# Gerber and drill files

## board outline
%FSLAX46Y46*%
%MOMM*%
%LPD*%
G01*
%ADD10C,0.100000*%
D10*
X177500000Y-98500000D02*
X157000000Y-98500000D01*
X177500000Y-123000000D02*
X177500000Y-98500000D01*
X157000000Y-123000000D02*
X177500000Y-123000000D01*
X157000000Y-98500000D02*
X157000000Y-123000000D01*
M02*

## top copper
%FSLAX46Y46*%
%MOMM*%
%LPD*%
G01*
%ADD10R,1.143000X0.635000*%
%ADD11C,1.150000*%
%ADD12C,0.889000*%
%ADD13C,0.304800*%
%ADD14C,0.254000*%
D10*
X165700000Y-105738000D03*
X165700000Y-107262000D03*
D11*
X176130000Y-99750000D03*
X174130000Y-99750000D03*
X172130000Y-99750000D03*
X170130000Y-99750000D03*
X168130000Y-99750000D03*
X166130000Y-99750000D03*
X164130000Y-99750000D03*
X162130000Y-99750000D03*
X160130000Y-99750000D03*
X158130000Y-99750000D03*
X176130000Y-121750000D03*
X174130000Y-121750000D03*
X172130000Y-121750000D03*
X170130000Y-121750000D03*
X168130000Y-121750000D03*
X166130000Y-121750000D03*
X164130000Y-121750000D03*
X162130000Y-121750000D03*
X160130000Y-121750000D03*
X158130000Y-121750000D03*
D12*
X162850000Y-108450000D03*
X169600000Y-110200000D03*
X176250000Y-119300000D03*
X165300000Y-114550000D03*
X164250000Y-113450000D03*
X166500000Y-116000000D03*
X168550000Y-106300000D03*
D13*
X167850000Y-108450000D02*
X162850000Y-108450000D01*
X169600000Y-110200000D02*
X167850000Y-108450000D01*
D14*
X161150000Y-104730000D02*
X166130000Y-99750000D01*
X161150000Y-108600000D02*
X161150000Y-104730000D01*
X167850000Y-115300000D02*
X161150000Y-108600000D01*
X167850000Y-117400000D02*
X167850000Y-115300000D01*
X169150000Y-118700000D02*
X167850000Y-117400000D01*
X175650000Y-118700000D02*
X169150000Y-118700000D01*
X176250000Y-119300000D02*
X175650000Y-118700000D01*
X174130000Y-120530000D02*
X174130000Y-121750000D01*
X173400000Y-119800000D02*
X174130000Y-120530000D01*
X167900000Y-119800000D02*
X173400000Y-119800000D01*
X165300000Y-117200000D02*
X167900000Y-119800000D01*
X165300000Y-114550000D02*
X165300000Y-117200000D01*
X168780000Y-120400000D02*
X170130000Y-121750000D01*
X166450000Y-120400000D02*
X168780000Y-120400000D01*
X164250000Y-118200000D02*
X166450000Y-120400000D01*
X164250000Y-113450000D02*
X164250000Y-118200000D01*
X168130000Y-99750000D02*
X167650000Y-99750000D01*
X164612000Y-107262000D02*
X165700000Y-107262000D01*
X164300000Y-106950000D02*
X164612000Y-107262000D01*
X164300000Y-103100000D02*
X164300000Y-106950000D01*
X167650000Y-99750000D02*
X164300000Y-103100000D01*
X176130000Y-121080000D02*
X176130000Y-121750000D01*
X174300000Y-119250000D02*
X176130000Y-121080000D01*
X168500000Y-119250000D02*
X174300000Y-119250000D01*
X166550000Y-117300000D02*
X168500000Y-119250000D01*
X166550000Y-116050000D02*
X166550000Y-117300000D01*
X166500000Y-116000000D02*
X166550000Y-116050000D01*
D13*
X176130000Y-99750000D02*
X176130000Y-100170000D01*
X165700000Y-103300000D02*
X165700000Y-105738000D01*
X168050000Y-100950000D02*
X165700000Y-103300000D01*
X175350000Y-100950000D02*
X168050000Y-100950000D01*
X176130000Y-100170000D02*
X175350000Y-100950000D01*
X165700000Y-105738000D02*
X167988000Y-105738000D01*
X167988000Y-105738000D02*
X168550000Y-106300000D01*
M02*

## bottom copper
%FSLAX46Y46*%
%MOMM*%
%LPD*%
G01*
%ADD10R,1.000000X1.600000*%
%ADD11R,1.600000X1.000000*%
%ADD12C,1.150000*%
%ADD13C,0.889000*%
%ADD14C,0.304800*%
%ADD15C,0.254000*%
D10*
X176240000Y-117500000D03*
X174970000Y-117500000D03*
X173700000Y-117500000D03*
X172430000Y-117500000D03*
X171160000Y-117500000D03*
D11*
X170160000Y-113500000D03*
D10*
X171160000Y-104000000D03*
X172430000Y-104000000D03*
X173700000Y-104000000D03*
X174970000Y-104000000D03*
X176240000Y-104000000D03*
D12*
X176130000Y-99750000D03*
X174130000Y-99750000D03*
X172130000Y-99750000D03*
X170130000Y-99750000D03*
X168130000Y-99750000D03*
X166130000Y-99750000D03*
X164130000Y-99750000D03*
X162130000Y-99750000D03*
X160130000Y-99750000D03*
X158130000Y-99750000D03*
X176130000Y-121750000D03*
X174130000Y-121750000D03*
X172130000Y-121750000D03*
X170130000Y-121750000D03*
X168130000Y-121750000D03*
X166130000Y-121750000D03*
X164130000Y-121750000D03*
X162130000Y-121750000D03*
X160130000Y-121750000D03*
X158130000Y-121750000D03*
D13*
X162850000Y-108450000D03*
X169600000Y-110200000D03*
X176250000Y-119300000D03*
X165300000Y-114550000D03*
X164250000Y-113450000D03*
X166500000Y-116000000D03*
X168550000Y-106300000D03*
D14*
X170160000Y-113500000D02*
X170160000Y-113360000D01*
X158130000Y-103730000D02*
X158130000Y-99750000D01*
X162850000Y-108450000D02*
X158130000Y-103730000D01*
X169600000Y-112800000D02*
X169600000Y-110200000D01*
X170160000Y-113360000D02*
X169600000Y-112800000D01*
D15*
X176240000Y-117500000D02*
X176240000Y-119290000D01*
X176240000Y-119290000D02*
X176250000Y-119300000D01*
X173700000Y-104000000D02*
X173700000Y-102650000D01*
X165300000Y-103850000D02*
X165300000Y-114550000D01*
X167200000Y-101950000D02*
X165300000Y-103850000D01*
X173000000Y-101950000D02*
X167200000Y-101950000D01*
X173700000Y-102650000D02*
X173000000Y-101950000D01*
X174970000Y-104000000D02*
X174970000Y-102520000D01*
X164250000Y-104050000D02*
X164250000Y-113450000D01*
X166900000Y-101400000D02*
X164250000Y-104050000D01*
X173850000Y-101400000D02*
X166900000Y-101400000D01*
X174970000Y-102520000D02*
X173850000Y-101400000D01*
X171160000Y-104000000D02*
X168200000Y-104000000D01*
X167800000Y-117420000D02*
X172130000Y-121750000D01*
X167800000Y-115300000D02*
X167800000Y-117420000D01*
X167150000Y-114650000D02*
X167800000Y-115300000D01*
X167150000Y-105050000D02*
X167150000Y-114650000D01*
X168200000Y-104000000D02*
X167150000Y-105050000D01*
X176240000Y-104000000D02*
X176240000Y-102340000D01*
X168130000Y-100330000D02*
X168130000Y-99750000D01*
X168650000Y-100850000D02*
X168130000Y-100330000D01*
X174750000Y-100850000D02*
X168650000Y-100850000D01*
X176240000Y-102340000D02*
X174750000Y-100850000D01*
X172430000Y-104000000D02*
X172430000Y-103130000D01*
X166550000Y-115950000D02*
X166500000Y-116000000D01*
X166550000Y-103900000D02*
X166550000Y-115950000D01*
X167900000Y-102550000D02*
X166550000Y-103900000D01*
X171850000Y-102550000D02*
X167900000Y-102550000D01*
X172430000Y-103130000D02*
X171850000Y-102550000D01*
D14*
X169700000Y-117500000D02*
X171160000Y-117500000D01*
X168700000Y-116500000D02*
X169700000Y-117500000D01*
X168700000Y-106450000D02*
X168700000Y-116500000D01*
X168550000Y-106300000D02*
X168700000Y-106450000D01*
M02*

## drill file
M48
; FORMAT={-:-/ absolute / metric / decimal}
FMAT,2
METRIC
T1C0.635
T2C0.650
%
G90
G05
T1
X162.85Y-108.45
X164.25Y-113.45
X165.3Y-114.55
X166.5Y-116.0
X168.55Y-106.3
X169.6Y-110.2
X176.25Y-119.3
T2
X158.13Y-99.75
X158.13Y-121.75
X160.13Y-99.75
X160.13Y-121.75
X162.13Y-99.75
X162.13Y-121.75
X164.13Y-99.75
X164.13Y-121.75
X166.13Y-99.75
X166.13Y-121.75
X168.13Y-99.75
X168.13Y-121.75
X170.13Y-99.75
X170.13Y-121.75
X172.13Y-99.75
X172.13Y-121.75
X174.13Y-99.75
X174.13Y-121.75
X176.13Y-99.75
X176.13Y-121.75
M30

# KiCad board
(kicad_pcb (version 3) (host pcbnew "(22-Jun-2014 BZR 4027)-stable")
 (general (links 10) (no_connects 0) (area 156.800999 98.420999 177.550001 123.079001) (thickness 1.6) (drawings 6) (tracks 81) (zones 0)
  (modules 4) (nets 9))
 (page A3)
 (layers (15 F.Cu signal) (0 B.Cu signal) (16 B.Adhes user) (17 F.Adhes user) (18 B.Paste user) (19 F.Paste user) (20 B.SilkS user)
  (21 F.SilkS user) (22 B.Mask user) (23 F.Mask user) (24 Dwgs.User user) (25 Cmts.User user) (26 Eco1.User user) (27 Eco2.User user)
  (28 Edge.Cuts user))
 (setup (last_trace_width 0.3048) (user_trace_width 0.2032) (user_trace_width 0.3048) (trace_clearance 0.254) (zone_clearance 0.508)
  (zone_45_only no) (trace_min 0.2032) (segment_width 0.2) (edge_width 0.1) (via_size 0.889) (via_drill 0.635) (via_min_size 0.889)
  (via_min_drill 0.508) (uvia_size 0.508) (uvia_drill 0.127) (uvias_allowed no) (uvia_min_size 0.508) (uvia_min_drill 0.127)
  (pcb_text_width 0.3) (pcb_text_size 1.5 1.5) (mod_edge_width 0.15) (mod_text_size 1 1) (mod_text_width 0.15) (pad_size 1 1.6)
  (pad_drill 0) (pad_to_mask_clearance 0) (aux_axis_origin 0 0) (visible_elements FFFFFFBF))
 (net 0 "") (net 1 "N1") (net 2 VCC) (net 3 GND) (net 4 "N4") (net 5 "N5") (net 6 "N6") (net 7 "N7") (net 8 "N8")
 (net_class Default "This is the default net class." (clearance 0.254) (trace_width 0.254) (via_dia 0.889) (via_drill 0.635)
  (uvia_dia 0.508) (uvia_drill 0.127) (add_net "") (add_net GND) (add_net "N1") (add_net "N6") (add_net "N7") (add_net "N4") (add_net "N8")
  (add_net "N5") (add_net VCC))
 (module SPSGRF (layer B.Cu) (at 173.7 110.75 90) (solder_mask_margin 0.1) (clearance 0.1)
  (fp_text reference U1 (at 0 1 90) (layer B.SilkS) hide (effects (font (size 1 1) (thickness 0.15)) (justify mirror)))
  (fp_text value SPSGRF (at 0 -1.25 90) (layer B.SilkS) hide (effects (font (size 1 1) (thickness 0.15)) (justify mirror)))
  (pad 1 smd rect (at -6.75 2.54 90) (size 1.6 1) (layers B.Cu B.Paste B.Mask) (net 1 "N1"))
  (pad 2 smd rect (at -6.75 1.27 90) (size 1.6 1) (layers B.Cu B.Paste B.Mask))
  (pad 3 smd rect (at -6.75 0 90) (size 1.6 1) (layers B.Cu B.Paste B.Mask))
  (pad 4 smd rect (at -6.75 -1.27 90) (size 1.6 1) (layers B.Cu B.Paste B.Mask))
  (pad 5 smd rect (at -6.75 -2.54 90) (size 1.6 1) (layers B.Cu B.Paste B.Mask) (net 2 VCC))
  (pad 6 smd rect (at -2.75 -3.54 90) (size 1 1.6) (layers B.Cu B.Paste B.Mask) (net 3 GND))
  (pad 7 smd rect (at 6.75 -2.54 90) (size 1.6 1) (layers B.Cu B.Paste B.Mask) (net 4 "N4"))
  (pad 8 smd rect (at 6.75 -1.27 90) (size 1.6 1) (layers B.Cu B.Paste B.Mask) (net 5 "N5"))
  (pad 9 smd rect (at 6.75 0 90) (size 1.6 1) (layers B.Cu B.Paste B.Mask) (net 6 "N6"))
  (pad 10 smd rect (at 6.75 1.27 90) (size 1.6 1) (layers B.Cu B.Paste B.Mask) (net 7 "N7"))
  (pad 11 smd rect (at 6.75 2.54 90) (size 1.6 1) (layers B.Cu B.Paste B.Mask) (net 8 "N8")))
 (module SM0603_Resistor (layer F.Cu) (at 165.7 106.5 270)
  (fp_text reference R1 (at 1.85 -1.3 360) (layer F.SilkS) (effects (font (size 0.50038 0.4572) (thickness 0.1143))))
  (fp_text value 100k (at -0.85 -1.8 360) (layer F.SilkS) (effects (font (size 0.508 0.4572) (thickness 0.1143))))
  (pad 1 smd rect (at -0.762 0 270) (size 0.635 1.143) (layers F.Cu F.Paste F.Mask) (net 2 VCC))
  (pad 2 smd rect (at 0.762 0 270) (size 0.635 1.143) (layers F.Cu F.Paste F.Mask) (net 8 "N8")))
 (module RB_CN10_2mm (layer F.Cu) (at 167.13 110.75)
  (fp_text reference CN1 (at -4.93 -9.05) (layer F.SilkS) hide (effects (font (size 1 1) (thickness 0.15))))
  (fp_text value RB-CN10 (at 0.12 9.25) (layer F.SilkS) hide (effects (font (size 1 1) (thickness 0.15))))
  (pad 1 thru_hole circle (at 9 -11) (size 1.15 1.15) (drill 0.65) (layers *.Cu *.Mask F.SilkS) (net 2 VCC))
  (pad 2 thru_hole circle (at 7 -11) (size 1.15 1.15) (drill 0.65) (layers *.Cu *.Mask F.SilkS))
  (pad 3 thru_hole circle (at 5 -11) (size 1.15 1.15) (drill 0.65) (layers *.Cu *.Mask F.SilkS))
  (pad 4 thru_hole circle (at 3 -11) (size 1.15 1.15) (drill 0.65) (layers *.Cu *.Mask F.SilkS))
  (pad 5 thru_hole circle (at 1 -11) (size 1.15 1.15) (drill 0.65) (layers *.Cu *.Mask F.SilkS) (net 8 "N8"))
  (pad 6 thru_hole circle (at -1 -11) (size 1.15 1.15) (drill 0.65) (layers *.Cu *.Mask F.SilkS) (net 1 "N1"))
  (pad 7 thru_hole circle (at -3 -11) (size 1.15 1.15) (drill 0.65) (layers *.Cu *.Mask F.SilkS))
  (pad 8 thru_hole circle (at -5 -11) (size 1.15 1.15) (drill 0.65) (layers *.Cu *.Mask F.SilkS))
  (pad 9 thru_hole circle (at -7 -11) (size 1.15 1.15) (drill 0.65) (layers *.Cu *.Mask F.SilkS))
  (pad 10 thru_hole circle (at -9 -11) (size 1.15 1.15) (drill 0.65) (layers *.Cu *.Mask F.SilkS) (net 3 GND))
  (pad 11 thru_hole circle (at 9 11) (size 1.15 1.15) (drill 0.65) (layers *.Cu *.Mask F.SilkS) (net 5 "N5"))
  (pad 12 thru_hole circle (at 7 11) (size 1.15 1.15) (drill 0.65) (layers *.Cu *.Mask F.SilkS) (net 6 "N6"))
  (pad 13 thru_hole circle (at 5 11) (size 1.15 1.15) (drill 0.65) (layers *.Cu *.Mask F.SilkS) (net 4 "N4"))
  (pad 14 thru_hole circle (at 3 11) (size 1.15 1.15) (drill 0.65) (layers *.Cu *.Mask F.SilkS) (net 7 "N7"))
  (pad 15 thru_hole circle (at 1 11) (size 1.15 1.15) (drill 0.65) (layers *.Cu *.Mask F.SilkS))
  (pad 16 thru_hole circle (at -1 11) (size 1.15 1.15) (drill 0.65) (layers *.Cu *.Mask F.SilkS))
  (pad 17 thru_hole circle (at -3 11) (size 1.15 1.15) (drill 0.65) (layers *.Cu *.Mask F.SilkS))
  (pad 18 thru_hole circle (at -5 11) (size 1.15 1.15) (drill 0.65) (layers *.Cu *.Mask F.SilkS))
  (pad 19 thru_hole circle (at -7 11) (size 1.15 1.15) (drill 0.65) (layers *.Cu *.Mask F.SilkS))
  (pad 20 thru_hole circle (at -9 11) (size 1.15 1.15) (drill 0.65) (layers *.Cu *.Mask F.SilkS)))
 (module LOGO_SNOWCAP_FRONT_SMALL (layer F.Cu) (at 172 110.95 270)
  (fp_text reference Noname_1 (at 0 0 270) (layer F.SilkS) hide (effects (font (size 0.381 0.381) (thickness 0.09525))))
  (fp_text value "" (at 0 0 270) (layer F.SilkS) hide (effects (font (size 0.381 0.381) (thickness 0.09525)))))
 (gr_line (start 177.5 98.5) (end 157 98.5) (angle 90) (layer Edge.Cuts) (width 0.1))
 (gr_line (start 177.5 123) (end 177.5 98.5) (angle 90) (layer Edge.Cuts) (width 0.1))
 (gr_line (start 157 123) (end 177.5 123) (angle 90) (layer Edge.Cuts) (width 0.1))
 (gr_line (start 157 98.5) (end 157 123) (angle 90) (layer Edge.Cuts) (width 0.1))
 (segment (start 170.16 113.5) (end 170.16 113.36) (width 0.3048) (layer B.Cu) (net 3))
 (segment (start 158.13 103.73) (end 158.13 99.75) (width 0.3048) (layer B.Cu) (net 3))
 (segment (start 162.85 108.45) (end 158.13 103.73) (width 0.3048) (layer B.Cu) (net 3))
 (segment (start 167.85 108.45) (end 162.85 108.45) (width 0.3048) (layer F.Cu) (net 3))
 (segment (start 169.6 110.2) (end 167.85 108.45) (width 0.3048) (layer F.Cu) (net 3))
 (segment (start 169.6 112.8) (end 169.6 110.2) (width 0.3048) (layer B.Cu) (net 3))
 (segment (start 170.16 113.36) (end 169.6 112.8) (width 0.3048) (layer B.Cu) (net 3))
 (segment (start 176.24 117.5) (end 176.24 119.29) (width 0.254) (layer B.Cu) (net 1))
 (segment (start 161.15 104.73) (end 166.13 99.75) (width 0.254) (layer F.Cu) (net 1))
 (segment (start 161.15 108.6) (end 161.15 104.73) (width 0.254) (layer F.Cu) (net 1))
 (segment (start 167.85 115.3) (end 161.15 108.6) (width 0.254) (layer F.Cu) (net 1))
 (segment (start 167.85 117.4) (end 167.85 115.3) (width 0.254) (layer F.Cu) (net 1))
 (segment (start 169.15 118.7) (end 167.85 117.4) (width 0.254) (layer F.Cu) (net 1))
 (segment (start 175.65 118.7) (end 169.15 118.7) (width 0.254) (layer F.Cu) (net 1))
 (segment (start 176.25 119.3) (end 175.65 118.7) (width 0.254) (layer F.Cu) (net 1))
 (segment (start 176.24 119.29) (end 176.25 119.3) (width 0.254) (layer B.Cu) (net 1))
 (segment (start 173.7 104) (end 173.7 102.65) (width 0.254) (layer B.Cu) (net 6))
 (segment (start 174.13 120.53) (end 174.13 121.75) (width 0.254) (layer F.Cu) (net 6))
 (segment (start 173.4 119.8) (end 174.13 120.53) (width 0.254) (layer F.Cu) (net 6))
 (segment (start 167.9 119.8) (end 173.4 119.8) (width 0.254) (layer F.Cu) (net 6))
 (segment (start 165.3 117.2) (end 167.9 119.8) (width 0.254) (layer F.Cu) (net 6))
 (segment (start 165.3 114.55) (end 165.3 117.2) (width 0.254) (layer F.Cu) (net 6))
 (segment (start 165.3 103.85) (end 165.3 114.55) (width 0.254) (layer B.Cu) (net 6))
 (segment (start 167.2 101.95) (end 165.3 103.85) (width 0.254) (layer B.Cu) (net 6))
 (segment (start 173 101.95) (end 167.2 101.95) (width 0.254) (layer B.Cu) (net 6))
 (segment (start 173.7 102.65) (end 173 101.95) (width 0.254) (layer B.Cu) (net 6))
 (segment (start 174.97 104) (end 174.97 102.52) (width 0.254) (layer B.Cu) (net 7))
 (segment (start 168.78 120.4) (end 170.13 121.75) (width 0.254) (layer F.Cu) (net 7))
 (segment (start 166.45 120.4) (end 168.78 120.4) (width 0.254) (layer F.Cu) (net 7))
 (segment (start 164.25 118.2) (end 166.45 120.4) (width 0.254) (layer F.Cu) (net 7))
 (segment (start 164.25 113.45) (end 164.25 118.2) (width 0.254) (layer F.Cu) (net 7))
 (segment (start 164.25 104.05) (end 164.25 113.45) (width 0.254) (layer B.Cu) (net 7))
 (segment (start 166.9 101.4) (end 164.25 104.05) (width 0.254) (layer B.Cu) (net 7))
 (segment (start 173.85 101.4) (end 166.9 101.4) (width 0.254) (layer B.Cu) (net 7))
 (segment (start 174.97 102.52) (end 173.85 101.4) (width 0.254) (layer B.Cu) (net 7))
 (segment (start 171.16 104) (end 168.2 104) (width 0.254) (layer B.Cu) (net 4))
 (segment (start 167.8 117.42) (end 172.13 121.75) (width 0.254) (layer B.Cu) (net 4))
 (segment (start 167.8 115.3) (end 167.8 117.42) (width 0.254) (layer B.Cu) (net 4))
 (segment (start 167.15 114.65) (end 167.8 115.3) (width 0.254) (layer B.Cu) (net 4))
 (segment (start 167.15 105.05) (end 167.15 114.65) (width 0.254) (layer B.Cu) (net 4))
 (segment (start 168.2 104) (end 167.15 105.05) (width 0.254) (layer B.Cu) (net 4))
 (segment (start 168.13 99.75) (end 167.65 99.75) (width 0.254) (layer F.Cu) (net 8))
 (segment (start 164.612 107.262) (end 165.7 107.262) (width 0.254) (layer F.Cu) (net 8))
 (segment (start 164.3 106.95) (end 164.612 107.262) (width 0.254) (layer F.Cu) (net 8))
 (segment (start 164.3 103.1) (end 164.3 106.95) (width 0.254) (layer F.Cu) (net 8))
 (segment (start 167.65 99.75) (end 164.3 103.1) (width 0.254) (layer F.Cu) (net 8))
 (segment (start 176.24 104) (end 176.24 102.34) (width 0.254) (layer B.Cu) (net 8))
 (segment (start 168.13 100.33) (end 168.13 99.75) (width 0.254) (layer B.Cu) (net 8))
 (segment (start 168.65 100.85) (end 168.13 100.33) (width 0.254) (layer B.Cu) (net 8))
 (segment (start 174.75 100.85) (end 168.65 100.85) (width 0.254) (layer B.Cu) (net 8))
 (segment (start 176.24 102.34) (end 174.75 100.85) (width 0.254) (layer B.Cu) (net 8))
 (segment (start 172.43 104) (end 172.43 103.13) (width 0.254) (layer B.Cu) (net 5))
 (segment (start 176.13 121.08) (end 176.13 121.75) (width 0.254) (layer F.Cu) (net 5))
 (segment (start 174.3 119.25) (end 176.13 121.08) (width 0.254) (layer F.Cu) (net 5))
 (segment (start 168.5 119.25) (end 174.3 119.25) (width 0.254) (layer F.Cu) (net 5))
 (segment (start 166.55 117.3) (end 168.5 119.25) (width 0.254) (layer F.Cu) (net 5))
 (segment (start 166.55 116.05) (end 166.55 117.3) (width 0.254) (layer F.Cu) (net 5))
 (segment (start 166.5 116) (end 166.55 116.05) (width 0.254) (layer F.Cu) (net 5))
 (segment (start 166.55 115.95) (end 166.5 116) (width 0.254) (layer B.Cu) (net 5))
 (segment (start 166.55 103.9) (end 166.55 115.95) (width 0.254) (layer B.Cu) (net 5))
 (segment (start 167.9 102.55) (end 166.55 103.9) (width 0.254) (layer B.Cu) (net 5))
 (segment (start 171.85 102.55) (end 167.9 102.55) (width 0.254) (layer B.Cu) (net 5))
 (segment (start 172.43 103.13) (end 171.85 102.55) (width 0.254) (layer B.Cu) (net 5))
 (segment (start 176.13 99.75) (end 176.13 100.17) (width 0.3048) (layer F.Cu) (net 2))
 (segment (start 165.7 103.3) (end 165.7 105.738) (width 0.3048) (layer F.Cu) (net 2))
 (segment (start 168.05 100.95) (end 165.7 103.3) (width 0.3048) (layer F.Cu) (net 2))
 (segment (start 175.35 100.95) (end 168.05 100.95) (width 0.3048) (layer F.Cu) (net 2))
 (segment (start 176.13 100.17) (end 175.35 100.95) (width 0.3048) (layer F.Cu) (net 2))
 (segment (start 165.7 105.738) (end 167.988 105.738) (width 0.3048) (layer F.Cu) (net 2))
 (segment (start 169.7 117.5) (end 171.16 117.5) (width 0.3048) (layer B.Cu) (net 2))
 (segment (start 168.7 116.5) (end 169.7 117.5) (width 0.3048) (layer B.Cu) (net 2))
 (segment (start 168.7 106.45) (end 168.7 116.5) (width 0.3048) (layer B.Cu) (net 2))
 (segment (start 168.55 106.3) (end 168.7 106.45) (width 0.3048) (layer B.Cu) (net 2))
 (segment (start 167.988 105.738) (end 168.55 106.3) (width 0.3048) (layer F.Cu) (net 2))
 (via (at 162.85 108.45) (size 0.889) (layers F.Cu B.Cu) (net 3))
 (via (at 169.6 110.2) (size 0.889) (layers F.Cu B.Cu) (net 3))
 (via (at 176.25 119.3) (size 0.889) (layers F.Cu B.Cu) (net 1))
 (via (at 165.3 114.55) (size 0.889) (layers F.Cu B.Cu) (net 6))
 (via (at 164.25 113.45) (size 0.889) (layers F.Cu B.Cu) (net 7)) (via (at 166.5 116) (size 0.889) (layers F.Cu B.Cu) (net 5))
 (via (at 168.55 106.3) (size 0.889) (layers F.Cu B.Cu) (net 2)))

